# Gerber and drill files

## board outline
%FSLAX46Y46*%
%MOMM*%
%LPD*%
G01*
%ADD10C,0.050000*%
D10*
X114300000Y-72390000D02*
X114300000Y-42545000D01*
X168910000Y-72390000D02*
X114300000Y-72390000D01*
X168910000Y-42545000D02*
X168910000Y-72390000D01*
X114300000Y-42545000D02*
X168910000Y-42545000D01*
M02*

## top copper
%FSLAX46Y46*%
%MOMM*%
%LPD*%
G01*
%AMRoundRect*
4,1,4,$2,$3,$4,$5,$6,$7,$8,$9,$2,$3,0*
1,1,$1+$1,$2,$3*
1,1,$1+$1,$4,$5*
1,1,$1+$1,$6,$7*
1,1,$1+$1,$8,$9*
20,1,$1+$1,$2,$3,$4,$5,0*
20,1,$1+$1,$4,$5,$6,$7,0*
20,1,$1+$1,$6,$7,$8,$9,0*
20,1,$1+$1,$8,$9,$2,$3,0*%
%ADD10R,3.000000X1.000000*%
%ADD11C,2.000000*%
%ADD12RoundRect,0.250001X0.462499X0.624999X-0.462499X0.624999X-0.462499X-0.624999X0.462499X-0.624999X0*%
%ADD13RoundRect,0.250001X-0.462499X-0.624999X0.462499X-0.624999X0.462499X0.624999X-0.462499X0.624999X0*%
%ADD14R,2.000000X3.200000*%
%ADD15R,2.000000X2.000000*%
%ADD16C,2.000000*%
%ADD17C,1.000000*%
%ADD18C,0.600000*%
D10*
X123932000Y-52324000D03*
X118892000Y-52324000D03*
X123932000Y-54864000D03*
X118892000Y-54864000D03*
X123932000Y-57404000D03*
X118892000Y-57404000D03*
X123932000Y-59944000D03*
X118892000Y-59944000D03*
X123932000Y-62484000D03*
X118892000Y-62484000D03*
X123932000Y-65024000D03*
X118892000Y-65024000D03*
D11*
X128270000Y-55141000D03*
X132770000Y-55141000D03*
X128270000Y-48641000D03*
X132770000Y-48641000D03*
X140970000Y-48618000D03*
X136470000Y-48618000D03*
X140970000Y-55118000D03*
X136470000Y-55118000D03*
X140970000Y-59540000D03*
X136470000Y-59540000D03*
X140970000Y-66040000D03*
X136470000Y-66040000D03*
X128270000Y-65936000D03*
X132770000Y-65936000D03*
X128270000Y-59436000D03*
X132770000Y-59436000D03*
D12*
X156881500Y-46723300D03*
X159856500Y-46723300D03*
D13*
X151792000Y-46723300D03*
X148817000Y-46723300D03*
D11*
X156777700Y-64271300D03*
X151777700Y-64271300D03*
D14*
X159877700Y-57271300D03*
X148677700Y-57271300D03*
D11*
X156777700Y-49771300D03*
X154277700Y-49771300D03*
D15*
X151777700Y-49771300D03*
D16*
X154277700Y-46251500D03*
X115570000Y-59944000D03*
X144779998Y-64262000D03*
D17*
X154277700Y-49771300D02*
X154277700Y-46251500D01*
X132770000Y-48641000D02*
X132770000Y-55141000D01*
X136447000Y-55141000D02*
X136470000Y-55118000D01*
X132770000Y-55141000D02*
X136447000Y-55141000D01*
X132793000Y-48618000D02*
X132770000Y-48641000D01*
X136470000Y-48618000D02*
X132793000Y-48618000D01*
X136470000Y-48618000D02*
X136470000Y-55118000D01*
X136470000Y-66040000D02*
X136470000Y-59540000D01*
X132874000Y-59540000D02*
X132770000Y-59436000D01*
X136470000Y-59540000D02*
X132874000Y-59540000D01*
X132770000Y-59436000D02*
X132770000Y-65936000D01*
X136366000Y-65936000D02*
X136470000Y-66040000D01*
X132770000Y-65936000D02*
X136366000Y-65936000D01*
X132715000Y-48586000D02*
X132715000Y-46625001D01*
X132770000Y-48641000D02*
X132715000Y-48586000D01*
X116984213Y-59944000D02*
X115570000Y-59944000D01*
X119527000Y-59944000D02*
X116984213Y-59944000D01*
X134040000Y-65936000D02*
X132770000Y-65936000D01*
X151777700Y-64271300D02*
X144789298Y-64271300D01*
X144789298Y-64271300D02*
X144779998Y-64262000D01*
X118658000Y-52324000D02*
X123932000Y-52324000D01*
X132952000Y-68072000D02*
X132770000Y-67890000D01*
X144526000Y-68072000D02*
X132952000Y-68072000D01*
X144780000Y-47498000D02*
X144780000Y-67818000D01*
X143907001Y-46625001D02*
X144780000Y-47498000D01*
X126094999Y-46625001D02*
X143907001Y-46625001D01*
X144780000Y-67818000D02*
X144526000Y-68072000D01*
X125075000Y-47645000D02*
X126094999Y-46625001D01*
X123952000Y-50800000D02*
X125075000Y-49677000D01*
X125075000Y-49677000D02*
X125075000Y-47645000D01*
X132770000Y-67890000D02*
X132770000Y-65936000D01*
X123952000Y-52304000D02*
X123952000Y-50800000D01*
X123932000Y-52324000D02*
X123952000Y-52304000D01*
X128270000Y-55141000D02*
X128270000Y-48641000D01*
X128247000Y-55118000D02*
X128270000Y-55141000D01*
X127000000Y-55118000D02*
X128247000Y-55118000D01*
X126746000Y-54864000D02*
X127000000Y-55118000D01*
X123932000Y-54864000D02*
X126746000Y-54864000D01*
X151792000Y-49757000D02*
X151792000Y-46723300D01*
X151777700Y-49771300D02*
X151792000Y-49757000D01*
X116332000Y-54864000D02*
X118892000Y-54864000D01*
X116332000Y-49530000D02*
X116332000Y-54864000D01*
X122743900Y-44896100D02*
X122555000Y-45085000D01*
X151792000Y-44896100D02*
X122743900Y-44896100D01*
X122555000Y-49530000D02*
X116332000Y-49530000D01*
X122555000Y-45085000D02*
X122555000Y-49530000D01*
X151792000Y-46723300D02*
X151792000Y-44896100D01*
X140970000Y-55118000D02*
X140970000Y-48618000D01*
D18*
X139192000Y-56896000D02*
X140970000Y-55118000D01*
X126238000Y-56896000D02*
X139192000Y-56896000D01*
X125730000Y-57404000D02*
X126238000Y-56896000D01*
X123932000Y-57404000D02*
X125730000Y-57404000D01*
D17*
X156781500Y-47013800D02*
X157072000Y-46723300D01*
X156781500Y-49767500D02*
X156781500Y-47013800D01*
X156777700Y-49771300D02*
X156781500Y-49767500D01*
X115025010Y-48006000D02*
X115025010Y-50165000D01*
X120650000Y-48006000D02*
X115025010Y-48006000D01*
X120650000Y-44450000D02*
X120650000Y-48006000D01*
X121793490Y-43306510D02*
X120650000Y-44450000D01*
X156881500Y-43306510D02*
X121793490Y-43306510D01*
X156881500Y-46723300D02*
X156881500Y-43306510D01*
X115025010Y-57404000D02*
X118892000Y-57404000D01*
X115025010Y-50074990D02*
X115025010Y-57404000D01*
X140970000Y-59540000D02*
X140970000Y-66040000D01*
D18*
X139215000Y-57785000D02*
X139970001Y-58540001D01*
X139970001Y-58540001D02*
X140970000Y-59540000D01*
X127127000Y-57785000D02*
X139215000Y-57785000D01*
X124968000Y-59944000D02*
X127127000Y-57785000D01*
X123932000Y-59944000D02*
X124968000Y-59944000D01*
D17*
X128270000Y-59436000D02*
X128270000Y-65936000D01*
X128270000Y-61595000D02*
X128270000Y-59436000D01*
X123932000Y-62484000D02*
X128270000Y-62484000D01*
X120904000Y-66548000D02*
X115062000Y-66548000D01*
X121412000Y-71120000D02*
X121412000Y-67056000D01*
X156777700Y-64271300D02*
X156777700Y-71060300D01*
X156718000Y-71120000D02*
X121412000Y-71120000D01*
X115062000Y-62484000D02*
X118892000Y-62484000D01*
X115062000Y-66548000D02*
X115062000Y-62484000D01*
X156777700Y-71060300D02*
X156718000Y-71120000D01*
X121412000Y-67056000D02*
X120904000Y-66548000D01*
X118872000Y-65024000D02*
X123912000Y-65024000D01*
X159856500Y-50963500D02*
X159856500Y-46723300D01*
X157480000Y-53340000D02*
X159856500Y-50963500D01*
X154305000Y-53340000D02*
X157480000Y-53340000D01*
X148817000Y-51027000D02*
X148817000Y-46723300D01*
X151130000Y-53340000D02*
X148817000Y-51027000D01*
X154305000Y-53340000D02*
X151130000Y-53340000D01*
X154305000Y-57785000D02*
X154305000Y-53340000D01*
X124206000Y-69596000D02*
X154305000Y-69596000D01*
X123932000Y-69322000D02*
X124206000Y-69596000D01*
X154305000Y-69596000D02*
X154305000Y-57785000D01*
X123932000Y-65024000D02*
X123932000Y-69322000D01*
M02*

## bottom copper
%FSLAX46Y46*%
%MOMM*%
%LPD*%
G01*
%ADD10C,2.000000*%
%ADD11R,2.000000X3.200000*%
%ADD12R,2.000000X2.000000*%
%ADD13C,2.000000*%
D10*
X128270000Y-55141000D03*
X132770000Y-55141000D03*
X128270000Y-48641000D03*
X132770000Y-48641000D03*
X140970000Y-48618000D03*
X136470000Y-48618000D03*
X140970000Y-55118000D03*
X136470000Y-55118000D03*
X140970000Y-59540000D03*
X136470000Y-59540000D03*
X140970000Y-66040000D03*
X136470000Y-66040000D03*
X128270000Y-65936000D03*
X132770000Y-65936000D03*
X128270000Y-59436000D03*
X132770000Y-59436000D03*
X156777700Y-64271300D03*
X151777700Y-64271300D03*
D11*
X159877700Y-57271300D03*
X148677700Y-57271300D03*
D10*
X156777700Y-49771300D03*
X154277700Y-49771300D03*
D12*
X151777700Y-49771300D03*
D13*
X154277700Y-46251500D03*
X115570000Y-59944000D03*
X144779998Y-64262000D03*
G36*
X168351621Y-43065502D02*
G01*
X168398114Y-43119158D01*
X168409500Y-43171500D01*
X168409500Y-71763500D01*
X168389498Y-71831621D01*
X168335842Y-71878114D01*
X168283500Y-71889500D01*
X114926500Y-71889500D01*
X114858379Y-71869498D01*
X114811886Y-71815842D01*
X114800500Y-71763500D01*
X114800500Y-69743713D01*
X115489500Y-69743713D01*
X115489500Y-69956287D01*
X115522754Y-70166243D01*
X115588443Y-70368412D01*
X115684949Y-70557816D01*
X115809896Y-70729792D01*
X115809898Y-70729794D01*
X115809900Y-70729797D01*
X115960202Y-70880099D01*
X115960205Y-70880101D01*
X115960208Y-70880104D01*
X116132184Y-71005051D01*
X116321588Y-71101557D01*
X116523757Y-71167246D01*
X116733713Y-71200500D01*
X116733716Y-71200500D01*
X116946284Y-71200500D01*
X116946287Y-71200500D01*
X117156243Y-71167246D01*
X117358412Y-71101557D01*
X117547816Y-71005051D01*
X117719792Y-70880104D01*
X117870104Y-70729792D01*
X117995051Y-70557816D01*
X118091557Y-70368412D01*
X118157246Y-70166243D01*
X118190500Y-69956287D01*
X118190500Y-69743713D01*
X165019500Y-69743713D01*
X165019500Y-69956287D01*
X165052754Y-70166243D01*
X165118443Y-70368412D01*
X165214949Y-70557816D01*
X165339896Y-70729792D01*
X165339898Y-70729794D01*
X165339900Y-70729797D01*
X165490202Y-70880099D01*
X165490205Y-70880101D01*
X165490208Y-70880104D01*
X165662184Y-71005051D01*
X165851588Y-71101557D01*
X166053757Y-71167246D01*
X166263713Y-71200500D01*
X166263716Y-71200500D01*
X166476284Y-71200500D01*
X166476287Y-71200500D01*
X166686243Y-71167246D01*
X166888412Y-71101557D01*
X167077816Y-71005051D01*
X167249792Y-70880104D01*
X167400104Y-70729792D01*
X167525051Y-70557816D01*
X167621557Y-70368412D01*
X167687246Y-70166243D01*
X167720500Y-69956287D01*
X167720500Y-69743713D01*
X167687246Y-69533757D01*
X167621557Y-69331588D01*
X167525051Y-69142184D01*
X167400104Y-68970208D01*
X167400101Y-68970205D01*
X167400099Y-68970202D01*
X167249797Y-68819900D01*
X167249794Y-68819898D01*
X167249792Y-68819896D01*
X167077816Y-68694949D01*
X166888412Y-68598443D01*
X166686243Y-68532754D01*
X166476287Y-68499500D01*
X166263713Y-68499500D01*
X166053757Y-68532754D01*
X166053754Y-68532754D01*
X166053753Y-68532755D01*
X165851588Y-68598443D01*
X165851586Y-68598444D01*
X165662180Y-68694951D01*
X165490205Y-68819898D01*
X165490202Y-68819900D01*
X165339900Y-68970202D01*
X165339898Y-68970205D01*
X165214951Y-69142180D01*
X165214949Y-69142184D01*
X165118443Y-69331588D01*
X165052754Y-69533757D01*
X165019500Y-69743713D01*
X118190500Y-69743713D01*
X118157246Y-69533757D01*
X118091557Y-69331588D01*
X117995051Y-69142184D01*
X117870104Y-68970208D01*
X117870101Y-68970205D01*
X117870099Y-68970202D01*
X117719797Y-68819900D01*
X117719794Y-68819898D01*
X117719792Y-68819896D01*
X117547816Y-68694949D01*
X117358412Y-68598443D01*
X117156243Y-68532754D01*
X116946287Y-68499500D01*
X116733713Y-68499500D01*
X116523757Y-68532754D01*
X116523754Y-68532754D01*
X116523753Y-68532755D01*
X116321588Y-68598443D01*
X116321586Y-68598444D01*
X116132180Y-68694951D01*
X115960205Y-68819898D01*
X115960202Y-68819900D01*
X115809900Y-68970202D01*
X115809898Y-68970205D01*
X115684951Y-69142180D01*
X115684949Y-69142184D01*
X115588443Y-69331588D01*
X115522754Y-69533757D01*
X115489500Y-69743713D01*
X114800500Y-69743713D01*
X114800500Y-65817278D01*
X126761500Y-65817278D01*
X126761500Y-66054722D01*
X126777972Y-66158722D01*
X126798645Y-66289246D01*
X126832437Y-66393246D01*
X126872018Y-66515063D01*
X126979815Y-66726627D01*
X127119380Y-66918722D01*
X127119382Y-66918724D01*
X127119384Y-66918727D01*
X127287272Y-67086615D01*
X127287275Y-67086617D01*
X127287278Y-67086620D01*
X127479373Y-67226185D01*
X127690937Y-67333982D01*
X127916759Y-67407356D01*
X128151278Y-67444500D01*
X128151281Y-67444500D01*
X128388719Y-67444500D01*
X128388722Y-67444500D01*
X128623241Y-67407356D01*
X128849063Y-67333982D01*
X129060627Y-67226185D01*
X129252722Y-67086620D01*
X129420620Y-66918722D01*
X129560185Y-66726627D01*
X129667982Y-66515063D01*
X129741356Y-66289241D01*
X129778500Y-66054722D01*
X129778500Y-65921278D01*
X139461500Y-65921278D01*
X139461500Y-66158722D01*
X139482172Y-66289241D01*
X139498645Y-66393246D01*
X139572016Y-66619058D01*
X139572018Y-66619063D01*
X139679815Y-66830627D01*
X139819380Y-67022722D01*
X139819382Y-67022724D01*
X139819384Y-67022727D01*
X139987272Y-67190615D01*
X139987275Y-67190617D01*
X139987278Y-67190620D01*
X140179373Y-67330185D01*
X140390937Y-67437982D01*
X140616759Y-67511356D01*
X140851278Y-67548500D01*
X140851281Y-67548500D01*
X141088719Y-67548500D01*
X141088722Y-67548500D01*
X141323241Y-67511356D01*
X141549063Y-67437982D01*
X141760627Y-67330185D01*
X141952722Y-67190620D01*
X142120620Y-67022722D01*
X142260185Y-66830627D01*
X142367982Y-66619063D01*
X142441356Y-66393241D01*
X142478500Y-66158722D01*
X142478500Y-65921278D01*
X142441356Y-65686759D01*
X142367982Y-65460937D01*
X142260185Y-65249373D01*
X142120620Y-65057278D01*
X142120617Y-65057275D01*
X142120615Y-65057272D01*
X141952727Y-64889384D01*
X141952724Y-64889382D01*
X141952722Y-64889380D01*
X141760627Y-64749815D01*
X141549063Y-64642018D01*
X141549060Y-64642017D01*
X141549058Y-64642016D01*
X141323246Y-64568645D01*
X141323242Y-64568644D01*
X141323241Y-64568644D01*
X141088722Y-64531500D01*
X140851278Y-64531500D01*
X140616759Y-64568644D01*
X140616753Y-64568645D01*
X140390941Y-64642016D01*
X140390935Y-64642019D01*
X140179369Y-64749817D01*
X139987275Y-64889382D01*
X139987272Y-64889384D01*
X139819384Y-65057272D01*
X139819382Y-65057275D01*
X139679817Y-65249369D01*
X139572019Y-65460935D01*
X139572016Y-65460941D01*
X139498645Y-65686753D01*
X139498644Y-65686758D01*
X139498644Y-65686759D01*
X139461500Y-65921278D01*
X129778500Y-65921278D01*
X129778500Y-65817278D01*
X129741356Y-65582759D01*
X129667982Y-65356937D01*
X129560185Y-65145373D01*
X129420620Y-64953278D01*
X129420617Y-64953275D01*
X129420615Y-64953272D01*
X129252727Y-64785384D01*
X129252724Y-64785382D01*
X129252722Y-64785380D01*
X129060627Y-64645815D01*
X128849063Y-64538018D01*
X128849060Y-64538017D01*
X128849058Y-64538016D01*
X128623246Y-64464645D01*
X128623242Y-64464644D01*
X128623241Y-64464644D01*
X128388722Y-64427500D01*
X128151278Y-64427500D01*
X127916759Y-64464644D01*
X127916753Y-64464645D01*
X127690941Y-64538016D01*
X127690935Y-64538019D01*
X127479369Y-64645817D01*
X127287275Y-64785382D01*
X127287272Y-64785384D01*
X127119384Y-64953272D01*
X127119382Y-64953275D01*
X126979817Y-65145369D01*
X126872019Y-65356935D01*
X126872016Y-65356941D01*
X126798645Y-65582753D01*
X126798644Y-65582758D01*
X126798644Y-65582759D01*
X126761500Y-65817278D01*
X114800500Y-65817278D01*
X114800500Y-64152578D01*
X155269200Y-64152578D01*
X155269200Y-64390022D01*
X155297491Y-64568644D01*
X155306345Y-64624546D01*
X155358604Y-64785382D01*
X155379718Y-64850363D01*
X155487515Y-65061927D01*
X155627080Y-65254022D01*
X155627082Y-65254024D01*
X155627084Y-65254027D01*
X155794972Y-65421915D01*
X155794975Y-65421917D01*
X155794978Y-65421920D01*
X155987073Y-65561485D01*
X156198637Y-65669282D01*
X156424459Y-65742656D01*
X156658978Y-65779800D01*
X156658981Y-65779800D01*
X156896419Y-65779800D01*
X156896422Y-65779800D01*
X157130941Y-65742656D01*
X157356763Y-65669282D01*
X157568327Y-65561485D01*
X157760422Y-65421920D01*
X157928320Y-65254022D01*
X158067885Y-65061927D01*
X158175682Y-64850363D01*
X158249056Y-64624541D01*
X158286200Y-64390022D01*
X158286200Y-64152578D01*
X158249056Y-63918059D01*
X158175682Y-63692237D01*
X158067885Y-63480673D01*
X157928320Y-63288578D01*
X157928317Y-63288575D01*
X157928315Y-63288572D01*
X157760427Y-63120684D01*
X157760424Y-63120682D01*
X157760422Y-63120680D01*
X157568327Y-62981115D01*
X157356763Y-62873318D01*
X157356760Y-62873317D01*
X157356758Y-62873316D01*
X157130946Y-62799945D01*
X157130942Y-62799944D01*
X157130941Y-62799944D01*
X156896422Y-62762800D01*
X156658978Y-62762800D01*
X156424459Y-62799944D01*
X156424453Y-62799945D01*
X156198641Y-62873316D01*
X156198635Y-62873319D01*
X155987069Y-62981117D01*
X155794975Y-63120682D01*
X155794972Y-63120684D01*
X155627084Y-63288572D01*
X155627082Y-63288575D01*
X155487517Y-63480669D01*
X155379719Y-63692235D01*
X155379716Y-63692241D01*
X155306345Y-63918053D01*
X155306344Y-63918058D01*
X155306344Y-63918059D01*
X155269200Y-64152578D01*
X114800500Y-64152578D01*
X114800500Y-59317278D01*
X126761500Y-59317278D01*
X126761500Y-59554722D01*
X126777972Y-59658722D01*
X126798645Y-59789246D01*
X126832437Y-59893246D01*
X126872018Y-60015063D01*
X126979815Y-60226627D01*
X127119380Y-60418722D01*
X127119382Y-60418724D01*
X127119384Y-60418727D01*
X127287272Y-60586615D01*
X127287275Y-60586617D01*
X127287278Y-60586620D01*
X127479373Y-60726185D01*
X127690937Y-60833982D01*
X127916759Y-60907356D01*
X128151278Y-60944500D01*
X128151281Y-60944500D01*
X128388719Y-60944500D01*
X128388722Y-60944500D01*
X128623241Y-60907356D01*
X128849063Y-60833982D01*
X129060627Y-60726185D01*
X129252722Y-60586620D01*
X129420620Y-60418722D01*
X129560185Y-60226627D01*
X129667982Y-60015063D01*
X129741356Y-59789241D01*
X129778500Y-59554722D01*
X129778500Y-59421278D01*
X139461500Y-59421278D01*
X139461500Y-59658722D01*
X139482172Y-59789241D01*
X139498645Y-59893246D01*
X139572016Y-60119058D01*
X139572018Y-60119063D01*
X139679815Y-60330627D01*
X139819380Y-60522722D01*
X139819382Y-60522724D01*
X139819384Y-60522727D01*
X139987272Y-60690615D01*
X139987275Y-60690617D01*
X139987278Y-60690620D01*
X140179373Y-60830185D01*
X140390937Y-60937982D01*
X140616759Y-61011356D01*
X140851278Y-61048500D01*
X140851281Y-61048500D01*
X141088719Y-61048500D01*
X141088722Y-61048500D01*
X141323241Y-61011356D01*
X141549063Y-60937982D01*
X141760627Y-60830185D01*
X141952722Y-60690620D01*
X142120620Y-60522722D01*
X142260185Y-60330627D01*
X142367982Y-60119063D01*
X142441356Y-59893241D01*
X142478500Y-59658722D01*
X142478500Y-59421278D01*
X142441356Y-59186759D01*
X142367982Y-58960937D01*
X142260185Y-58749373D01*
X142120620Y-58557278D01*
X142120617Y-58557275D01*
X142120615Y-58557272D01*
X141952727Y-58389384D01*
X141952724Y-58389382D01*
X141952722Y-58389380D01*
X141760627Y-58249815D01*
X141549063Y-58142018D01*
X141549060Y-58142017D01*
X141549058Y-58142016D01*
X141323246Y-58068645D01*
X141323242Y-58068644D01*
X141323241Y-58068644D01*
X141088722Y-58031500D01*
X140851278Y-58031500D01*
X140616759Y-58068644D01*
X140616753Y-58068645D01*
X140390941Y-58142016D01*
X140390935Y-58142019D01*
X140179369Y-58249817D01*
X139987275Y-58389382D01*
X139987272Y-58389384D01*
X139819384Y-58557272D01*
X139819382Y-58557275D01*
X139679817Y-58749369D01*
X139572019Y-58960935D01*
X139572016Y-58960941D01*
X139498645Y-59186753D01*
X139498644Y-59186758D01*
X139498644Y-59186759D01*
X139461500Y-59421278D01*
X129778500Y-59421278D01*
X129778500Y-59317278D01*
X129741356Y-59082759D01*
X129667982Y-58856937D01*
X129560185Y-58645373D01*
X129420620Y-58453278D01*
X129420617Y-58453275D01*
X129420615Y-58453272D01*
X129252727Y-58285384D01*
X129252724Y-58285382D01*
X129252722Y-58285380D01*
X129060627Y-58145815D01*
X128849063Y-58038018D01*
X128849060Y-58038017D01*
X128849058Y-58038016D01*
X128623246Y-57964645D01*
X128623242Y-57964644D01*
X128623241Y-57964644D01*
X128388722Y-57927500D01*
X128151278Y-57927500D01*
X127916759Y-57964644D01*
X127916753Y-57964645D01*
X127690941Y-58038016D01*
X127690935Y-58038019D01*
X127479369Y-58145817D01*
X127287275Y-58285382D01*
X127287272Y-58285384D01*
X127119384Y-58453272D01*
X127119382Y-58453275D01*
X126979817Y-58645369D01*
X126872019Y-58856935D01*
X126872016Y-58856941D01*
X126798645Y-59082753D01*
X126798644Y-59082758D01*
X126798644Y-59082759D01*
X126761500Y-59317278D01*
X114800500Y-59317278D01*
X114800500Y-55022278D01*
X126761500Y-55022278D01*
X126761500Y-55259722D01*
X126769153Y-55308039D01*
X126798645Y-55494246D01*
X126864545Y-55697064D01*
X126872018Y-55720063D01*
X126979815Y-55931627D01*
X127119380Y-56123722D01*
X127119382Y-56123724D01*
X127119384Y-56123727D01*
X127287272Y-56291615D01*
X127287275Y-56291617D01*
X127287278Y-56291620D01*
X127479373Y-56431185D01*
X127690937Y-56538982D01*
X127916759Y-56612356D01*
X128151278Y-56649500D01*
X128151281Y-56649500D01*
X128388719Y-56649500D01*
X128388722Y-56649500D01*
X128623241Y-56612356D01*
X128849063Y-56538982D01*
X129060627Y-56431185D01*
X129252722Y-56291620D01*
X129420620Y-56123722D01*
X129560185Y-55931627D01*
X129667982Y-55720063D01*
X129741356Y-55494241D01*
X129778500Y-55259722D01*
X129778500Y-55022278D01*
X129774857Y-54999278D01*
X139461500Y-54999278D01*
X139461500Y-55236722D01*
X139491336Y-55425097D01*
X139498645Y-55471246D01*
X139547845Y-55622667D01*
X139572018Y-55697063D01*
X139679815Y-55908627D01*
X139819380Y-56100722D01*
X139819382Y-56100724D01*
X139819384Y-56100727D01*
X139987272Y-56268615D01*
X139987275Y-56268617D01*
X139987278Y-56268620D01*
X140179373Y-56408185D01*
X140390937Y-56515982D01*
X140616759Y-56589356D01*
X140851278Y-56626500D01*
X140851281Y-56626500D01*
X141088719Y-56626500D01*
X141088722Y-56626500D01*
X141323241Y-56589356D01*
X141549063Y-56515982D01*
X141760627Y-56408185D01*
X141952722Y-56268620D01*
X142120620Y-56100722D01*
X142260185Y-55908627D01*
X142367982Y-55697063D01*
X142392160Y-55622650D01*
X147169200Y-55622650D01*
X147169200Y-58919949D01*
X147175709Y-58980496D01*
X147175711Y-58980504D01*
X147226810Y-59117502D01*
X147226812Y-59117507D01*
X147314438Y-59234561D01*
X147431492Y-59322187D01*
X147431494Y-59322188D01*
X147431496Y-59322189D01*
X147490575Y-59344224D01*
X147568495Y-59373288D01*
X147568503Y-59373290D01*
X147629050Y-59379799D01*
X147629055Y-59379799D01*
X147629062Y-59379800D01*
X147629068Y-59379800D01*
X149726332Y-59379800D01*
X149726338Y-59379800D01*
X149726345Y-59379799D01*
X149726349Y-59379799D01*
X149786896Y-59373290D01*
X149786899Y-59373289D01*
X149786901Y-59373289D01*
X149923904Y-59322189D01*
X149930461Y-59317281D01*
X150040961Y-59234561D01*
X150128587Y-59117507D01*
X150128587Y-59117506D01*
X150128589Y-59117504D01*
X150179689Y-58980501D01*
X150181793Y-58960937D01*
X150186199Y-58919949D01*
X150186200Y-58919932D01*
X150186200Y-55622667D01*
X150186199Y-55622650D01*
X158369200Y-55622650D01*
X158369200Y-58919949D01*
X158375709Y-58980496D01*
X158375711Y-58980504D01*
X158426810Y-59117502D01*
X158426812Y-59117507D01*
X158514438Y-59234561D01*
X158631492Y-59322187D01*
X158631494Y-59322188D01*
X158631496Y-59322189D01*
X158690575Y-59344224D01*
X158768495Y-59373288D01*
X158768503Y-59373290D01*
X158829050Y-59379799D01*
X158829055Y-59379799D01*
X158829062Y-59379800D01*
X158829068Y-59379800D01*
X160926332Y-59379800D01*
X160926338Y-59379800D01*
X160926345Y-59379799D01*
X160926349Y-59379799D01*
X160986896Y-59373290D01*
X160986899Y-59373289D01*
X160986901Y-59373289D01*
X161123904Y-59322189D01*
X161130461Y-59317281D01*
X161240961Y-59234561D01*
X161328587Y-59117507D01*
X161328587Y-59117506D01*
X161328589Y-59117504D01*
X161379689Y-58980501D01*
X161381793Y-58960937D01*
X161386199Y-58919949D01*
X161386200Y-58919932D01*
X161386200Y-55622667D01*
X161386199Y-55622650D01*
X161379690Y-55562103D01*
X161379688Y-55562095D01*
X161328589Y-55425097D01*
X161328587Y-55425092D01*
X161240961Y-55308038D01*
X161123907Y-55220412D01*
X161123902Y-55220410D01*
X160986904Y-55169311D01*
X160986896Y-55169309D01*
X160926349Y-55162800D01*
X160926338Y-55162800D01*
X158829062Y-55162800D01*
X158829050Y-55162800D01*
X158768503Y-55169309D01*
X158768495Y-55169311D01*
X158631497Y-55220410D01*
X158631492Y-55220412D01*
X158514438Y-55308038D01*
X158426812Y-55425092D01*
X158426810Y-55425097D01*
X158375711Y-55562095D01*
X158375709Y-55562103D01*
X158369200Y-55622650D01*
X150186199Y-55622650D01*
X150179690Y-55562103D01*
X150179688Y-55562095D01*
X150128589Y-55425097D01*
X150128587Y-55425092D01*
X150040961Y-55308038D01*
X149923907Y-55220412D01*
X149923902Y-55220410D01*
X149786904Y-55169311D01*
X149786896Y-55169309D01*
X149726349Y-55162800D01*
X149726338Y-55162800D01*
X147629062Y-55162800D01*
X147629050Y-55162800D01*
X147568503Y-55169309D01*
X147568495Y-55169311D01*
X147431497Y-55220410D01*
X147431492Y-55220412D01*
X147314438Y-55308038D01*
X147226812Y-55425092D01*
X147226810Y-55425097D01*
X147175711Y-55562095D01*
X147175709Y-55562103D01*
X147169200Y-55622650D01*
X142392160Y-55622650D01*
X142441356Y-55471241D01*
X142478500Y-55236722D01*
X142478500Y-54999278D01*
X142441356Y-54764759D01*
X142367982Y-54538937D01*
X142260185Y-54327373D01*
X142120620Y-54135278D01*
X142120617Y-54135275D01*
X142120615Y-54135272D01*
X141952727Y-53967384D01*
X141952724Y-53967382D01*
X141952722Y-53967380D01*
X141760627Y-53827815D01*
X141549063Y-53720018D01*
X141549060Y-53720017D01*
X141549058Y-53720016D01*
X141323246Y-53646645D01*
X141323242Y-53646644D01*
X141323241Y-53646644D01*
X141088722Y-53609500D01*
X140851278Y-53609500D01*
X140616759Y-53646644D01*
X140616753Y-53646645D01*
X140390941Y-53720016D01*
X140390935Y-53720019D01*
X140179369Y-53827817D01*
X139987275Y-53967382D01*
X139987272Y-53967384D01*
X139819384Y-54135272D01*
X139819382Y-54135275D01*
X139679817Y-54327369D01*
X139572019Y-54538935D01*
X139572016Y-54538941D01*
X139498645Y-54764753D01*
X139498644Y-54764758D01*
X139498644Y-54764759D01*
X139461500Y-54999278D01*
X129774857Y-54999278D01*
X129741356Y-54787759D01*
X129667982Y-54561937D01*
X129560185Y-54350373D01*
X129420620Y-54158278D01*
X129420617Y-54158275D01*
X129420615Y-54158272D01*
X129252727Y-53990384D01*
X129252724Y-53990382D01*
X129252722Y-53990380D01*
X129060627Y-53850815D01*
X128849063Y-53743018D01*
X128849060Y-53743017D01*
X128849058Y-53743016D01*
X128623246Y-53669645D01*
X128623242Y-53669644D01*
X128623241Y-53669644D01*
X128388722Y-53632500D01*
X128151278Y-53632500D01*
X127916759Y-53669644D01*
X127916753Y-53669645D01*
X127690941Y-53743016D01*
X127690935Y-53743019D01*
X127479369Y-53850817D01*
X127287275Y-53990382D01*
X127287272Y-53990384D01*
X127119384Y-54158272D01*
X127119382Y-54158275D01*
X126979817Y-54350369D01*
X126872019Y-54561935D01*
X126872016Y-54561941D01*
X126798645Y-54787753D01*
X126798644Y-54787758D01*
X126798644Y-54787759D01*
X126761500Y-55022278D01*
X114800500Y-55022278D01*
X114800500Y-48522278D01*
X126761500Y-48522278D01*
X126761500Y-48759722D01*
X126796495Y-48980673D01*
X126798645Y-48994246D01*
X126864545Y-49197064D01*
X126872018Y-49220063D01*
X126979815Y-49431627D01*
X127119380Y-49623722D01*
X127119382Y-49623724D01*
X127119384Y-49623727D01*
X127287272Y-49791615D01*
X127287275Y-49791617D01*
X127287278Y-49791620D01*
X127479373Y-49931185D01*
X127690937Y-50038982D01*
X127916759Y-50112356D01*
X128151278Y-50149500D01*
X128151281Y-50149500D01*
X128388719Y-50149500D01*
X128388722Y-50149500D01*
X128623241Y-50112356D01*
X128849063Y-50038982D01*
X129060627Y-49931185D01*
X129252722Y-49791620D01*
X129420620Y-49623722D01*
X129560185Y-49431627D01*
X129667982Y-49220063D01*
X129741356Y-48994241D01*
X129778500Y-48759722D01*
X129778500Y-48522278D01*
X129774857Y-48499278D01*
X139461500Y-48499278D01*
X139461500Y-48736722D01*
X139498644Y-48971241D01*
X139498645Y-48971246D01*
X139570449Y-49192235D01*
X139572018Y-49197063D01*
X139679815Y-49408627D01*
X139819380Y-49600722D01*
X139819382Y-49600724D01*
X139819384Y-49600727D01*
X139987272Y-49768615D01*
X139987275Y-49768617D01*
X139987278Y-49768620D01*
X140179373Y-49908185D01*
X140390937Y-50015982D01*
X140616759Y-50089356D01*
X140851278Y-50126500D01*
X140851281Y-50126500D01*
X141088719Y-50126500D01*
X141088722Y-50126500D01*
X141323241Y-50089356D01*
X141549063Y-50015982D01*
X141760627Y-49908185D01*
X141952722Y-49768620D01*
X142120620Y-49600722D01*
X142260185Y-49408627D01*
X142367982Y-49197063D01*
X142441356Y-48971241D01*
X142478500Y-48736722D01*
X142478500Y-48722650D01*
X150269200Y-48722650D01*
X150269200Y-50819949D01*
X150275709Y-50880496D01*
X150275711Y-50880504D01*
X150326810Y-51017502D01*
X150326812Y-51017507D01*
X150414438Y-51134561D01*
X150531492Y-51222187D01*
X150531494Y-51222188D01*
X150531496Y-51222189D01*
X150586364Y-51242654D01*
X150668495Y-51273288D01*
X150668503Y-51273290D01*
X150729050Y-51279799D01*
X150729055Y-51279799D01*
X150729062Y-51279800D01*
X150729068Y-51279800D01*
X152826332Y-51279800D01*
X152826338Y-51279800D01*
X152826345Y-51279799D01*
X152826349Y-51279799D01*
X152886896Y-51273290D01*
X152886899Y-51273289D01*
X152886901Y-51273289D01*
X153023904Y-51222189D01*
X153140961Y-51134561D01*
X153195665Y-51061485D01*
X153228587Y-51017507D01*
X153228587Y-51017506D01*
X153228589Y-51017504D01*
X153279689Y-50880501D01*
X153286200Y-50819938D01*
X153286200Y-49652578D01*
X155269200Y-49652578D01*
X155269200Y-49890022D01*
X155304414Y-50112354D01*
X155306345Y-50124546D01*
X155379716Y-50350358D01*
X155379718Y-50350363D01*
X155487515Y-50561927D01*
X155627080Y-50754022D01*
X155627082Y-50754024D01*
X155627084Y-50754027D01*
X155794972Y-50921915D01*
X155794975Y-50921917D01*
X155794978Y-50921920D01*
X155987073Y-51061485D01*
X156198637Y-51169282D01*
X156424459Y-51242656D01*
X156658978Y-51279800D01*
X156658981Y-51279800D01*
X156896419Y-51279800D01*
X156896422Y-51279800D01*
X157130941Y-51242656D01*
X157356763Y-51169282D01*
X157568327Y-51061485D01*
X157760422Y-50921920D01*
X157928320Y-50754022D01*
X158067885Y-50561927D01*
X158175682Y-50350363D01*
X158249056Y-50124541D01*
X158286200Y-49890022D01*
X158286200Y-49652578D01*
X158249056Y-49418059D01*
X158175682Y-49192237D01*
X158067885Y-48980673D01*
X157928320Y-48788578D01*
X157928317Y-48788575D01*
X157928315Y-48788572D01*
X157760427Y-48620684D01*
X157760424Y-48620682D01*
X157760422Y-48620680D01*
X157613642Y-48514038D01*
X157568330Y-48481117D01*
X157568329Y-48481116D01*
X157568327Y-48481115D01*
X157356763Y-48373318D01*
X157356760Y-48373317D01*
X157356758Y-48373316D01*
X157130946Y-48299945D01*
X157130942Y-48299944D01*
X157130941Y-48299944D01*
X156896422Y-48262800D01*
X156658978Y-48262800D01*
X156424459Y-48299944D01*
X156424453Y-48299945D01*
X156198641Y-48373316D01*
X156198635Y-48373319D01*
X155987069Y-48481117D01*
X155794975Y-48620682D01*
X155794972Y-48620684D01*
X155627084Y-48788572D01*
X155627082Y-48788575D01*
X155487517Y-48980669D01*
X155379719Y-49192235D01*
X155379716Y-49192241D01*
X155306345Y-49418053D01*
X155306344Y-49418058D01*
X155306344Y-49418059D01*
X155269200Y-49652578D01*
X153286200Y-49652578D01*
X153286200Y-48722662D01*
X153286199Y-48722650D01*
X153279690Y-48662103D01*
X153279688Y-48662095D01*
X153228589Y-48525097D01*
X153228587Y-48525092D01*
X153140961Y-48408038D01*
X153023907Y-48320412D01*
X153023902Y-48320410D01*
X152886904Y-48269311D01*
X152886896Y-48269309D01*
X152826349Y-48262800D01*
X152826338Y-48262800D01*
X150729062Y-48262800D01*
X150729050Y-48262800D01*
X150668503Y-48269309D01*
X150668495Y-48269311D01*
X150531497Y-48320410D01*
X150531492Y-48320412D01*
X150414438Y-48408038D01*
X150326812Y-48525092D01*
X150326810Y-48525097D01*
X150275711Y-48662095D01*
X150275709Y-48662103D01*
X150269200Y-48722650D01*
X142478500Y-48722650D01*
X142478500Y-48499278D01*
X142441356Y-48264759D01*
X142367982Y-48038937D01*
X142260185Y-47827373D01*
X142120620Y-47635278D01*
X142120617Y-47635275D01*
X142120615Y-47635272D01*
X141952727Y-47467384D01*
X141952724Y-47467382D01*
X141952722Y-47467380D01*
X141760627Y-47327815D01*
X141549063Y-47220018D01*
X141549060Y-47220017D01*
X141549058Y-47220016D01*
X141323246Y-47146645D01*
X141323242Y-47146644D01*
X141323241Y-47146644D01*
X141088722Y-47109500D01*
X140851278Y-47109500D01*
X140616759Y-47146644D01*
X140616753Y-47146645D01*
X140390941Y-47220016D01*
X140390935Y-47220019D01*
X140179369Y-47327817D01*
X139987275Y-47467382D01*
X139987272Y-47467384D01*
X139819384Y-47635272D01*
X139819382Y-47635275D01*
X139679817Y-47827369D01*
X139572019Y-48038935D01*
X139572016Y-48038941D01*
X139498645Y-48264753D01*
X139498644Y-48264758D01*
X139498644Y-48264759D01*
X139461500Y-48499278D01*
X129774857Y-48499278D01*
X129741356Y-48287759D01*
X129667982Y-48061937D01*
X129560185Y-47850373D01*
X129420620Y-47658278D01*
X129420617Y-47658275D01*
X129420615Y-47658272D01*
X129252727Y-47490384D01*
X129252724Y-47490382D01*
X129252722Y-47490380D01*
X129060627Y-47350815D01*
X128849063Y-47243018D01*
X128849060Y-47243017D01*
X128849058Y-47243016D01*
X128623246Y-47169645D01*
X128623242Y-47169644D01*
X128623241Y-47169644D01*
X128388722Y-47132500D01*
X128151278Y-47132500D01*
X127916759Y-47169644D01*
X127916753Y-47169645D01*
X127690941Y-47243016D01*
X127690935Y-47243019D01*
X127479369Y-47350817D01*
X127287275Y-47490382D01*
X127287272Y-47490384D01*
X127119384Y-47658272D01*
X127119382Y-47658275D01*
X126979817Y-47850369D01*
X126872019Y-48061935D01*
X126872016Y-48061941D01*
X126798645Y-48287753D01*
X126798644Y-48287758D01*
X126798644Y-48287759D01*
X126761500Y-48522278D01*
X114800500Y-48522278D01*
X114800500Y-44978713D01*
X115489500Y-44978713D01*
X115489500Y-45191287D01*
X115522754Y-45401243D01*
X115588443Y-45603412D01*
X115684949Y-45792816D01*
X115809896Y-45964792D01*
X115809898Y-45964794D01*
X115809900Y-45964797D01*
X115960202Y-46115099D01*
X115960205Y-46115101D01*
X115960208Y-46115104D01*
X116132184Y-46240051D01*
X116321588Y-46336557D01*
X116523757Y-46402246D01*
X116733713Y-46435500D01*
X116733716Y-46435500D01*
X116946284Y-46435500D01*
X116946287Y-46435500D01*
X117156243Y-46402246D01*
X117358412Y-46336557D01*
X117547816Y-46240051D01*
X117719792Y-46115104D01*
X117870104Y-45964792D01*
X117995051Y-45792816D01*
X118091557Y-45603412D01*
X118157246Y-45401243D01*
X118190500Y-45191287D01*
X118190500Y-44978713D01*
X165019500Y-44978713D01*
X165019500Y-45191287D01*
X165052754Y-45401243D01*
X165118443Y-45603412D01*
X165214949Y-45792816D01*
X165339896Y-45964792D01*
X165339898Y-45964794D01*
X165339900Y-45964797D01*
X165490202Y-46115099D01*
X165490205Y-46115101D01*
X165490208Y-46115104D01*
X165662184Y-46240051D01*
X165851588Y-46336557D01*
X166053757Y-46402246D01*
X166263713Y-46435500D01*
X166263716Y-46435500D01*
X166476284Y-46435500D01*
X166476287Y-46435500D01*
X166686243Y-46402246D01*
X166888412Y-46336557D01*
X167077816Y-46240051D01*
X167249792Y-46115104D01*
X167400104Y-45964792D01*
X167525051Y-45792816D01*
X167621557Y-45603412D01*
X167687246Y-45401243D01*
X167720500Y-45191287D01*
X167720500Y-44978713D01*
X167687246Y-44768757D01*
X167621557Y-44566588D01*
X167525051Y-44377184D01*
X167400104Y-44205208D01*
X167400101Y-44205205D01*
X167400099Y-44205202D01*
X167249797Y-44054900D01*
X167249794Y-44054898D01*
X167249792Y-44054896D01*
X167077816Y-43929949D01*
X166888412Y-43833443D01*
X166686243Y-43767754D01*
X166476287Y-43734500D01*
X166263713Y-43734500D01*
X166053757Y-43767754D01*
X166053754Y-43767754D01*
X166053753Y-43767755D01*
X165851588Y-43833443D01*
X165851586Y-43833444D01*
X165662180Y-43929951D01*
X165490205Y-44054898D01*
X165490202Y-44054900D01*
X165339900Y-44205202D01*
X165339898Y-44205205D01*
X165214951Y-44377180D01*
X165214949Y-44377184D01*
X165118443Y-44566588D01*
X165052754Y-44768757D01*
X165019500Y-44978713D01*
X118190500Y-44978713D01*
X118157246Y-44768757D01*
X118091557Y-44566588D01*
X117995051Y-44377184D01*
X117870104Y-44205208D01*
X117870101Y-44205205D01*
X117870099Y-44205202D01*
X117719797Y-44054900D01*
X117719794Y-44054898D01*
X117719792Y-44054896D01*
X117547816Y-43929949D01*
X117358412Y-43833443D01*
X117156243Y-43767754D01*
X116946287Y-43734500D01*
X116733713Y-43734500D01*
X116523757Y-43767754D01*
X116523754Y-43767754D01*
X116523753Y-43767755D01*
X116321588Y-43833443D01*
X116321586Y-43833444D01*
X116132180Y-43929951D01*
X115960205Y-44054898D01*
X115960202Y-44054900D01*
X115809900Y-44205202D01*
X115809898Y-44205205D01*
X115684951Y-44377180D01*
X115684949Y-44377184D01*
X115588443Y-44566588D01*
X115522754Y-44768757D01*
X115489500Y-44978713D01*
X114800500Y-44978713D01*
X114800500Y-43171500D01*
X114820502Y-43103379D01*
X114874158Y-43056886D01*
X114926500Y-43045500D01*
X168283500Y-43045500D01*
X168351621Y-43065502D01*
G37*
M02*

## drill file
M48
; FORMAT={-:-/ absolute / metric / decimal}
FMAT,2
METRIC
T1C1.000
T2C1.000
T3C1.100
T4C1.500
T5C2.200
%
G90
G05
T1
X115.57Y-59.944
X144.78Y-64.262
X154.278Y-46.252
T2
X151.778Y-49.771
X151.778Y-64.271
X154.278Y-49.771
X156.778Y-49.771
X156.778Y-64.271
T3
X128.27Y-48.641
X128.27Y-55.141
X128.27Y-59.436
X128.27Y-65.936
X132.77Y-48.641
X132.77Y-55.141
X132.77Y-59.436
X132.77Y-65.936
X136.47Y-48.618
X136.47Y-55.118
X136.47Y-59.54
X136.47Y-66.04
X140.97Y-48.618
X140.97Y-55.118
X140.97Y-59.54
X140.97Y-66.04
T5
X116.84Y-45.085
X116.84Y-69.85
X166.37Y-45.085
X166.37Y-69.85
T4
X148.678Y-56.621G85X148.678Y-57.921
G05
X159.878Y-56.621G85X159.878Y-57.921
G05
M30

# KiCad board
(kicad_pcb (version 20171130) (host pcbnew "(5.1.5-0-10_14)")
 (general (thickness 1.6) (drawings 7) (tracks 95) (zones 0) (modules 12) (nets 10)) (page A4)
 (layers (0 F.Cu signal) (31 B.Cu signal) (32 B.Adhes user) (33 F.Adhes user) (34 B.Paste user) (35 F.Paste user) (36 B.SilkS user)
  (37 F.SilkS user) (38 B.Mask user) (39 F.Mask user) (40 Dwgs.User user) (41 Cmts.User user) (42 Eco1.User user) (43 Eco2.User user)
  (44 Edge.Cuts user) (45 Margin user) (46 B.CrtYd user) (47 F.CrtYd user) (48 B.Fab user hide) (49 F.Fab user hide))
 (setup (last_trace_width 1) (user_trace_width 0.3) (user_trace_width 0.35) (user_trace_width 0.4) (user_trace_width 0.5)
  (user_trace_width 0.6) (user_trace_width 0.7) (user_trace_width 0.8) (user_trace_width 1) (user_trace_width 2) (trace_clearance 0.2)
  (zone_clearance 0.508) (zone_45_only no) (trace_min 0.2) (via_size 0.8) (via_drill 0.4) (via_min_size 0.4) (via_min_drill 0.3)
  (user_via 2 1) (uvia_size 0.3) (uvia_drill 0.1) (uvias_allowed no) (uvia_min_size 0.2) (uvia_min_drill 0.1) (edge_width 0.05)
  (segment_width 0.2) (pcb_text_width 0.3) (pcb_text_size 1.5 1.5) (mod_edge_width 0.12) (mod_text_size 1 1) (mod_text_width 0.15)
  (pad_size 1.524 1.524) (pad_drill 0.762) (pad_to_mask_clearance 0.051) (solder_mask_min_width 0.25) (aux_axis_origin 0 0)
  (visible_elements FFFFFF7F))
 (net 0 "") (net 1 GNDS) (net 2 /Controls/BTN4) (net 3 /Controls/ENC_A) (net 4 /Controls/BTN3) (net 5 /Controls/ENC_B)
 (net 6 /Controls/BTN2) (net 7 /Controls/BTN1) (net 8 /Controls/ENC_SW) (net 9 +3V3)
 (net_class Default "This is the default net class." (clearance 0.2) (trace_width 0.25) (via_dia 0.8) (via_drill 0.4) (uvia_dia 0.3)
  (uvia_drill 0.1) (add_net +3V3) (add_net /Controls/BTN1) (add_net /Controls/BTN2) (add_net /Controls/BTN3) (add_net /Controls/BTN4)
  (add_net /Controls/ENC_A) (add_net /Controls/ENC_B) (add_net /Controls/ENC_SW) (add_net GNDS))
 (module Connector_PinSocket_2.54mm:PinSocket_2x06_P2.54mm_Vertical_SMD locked (layer F.Cu) (at 121.412 58.674 180)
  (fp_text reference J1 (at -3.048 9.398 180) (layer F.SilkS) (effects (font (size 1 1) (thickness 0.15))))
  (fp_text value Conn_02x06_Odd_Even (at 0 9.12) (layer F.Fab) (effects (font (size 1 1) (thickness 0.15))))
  (pad 12 smd rect (at -2.52 6.35 180) (size 3 1) (layers F.Cu F.Paste F.Mask) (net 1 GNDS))
  (pad 11 smd rect (at 2.52 6.35 180) (size 3 1) (layers F.Cu F.Paste F.Mask) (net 1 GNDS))
  (pad 10 smd rect (at -2.52 3.81 180) (size 3 1) (layers F.Cu F.Paste F.Mask) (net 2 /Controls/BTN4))
  (pad 9 smd rect (at 2.52 3.81 180) (size 3 1) (layers F.Cu F.Paste F.Mask) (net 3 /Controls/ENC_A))
  (pad 8 smd rect (at -2.52 1.27 180) (size 3 1) (layers F.Cu F.Paste F.Mask) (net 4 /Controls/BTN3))
  (pad 7 smd rect (at 2.52 1.27 180) (size 3 1) (layers F.Cu F.Paste F.Mask) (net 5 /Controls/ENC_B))
  (pad 6 smd rect (at -2.52 -1.27 180) (size 3 1) (layers F.Cu F.Paste F.Mask) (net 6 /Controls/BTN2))
  (pad 5 smd rect (at 2.52 -1.27 180) (size 3 1) (layers F.Cu F.Paste F.Mask) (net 1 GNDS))
  (pad 4 smd rect (at -2.52 -3.81 180) (size 3 1) (layers F.Cu F.Paste F.Mask) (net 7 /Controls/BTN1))
  (pad 3 smd rect (at 2.52 -3.81 180) (size 3 1) (layers F.Cu F.Paste F.Mask) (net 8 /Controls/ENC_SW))
  (pad 2 smd rect (at -2.52 -6.35 180) (size 3 1) (layers F.Cu F.Paste F.Mask) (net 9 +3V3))
  (pad 1 smd rect (at 2.52 -6.35 180) (size 3 1) (layers F.Cu F.Paste F.Mask) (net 9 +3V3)))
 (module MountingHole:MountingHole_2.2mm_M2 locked (layer F.Cu) (at 166.37 45.085)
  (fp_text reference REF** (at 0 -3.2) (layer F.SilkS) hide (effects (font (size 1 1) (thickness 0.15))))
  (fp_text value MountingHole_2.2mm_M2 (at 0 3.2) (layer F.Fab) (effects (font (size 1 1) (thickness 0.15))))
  (pad 1 np_thru_hole circle (at 0 0) (size 2.2 2.2) (drill 2.2) (layers *.Cu *.Mask)))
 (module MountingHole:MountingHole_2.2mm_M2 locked (layer F.Cu) (at 166.37 69.85)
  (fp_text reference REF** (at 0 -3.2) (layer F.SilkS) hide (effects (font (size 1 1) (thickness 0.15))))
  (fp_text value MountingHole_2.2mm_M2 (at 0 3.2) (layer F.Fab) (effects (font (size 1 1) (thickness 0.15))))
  (pad 1 np_thru_hole circle (at 0 0) (size 2.2 2.2) (drill 2.2) (layers *.Cu *.Mask)))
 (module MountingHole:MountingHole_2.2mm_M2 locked (layer F.Cu) (at 116.84 69.85)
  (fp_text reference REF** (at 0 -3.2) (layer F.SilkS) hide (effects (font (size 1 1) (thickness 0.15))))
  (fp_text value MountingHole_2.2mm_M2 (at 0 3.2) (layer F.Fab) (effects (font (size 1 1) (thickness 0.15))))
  (pad 1 np_thru_hole circle (at 0 0) (size 2.2 2.2) (drill 2.2) (layers *.Cu *.Mask)))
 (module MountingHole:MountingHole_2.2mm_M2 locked (layer F.Cu) (at 116.84 45.085)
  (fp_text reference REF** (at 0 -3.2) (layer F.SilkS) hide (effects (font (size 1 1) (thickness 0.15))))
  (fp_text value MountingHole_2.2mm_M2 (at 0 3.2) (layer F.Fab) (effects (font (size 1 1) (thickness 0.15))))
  (pad 1 np_thru_hole circle (at 0 0) (size 2.2 2.2) (drill 2.2) (layers *.Cu *.Mask)))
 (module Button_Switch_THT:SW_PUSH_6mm (layer B.Cu) (at 128.27 48.641 270)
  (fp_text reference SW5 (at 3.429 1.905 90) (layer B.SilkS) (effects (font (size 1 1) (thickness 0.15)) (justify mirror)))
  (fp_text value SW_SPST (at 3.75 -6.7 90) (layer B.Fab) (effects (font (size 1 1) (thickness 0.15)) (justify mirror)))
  (pad 1 thru_hole circle (at 6.5 0 180) (size 2 2) (drill 1.1) (layers *.Cu *.Mask) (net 2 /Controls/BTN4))
  (pad 2 thru_hole circle (at 6.5 -4.5 180) (size 2 2) (drill 1.1) (layers *.Cu *.Mask) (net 1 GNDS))
  (pad 1 thru_hole circle (at 0 0 180) (size 2 2) (drill 1.1) (layers *.Cu *.Mask) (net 2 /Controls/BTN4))
  (pad 2 thru_hole circle (at 0 -4.5 180) (size 2 2) (drill 1.1) (layers *.Cu *.Mask) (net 1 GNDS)))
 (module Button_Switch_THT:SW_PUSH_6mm (layer B.Cu) (at 140.97 55.118 90)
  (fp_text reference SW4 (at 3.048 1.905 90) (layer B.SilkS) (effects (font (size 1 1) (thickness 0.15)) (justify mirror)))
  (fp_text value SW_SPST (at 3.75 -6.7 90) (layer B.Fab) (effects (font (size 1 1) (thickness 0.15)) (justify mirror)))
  (pad 1 thru_hole circle (at 6.5 0) (size 2 2) (drill 1.1) (layers *.Cu *.Mask) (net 4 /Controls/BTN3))
  (pad 2 thru_hole circle (at 6.5 -4.5) (size 2 2) (drill 1.1) (layers *.Cu *.Mask) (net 1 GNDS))
  (pad 1 thru_hole circle (at 0 0) (size 2 2) (drill 1.1) (layers *.Cu *.Mask) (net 4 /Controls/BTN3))
  (pad 2 thru_hole circle (at 0 -4.5) (size 2 2) (drill 1.1) (layers *.Cu *.Mask) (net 1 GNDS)))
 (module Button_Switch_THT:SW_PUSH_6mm (layer B.Cu) (at 140.97 66.04 90)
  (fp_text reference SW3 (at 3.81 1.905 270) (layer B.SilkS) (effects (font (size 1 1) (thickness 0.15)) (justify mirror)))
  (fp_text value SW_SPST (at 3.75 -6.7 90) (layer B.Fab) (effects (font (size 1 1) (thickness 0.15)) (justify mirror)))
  (pad 1 thru_hole circle (at 6.5 0) (size 2 2) (drill 1.1) (layers *.Cu *.Mask) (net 6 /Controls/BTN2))
  (pad 2 thru_hole circle (at 6.5 -4.5) (size 2 2) (drill 1.1) (layers *.Cu *.Mask) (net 1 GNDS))
  (pad 1 thru_hole circle (at 0 0) (size 2 2) (drill 1.1) (layers *.Cu *.Mask) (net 6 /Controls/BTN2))
  (pad 2 thru_hole circle (at 0 -4.5) (size 2 2) (drill 1.1) (layers *.Cu *.Mask) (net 1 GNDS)))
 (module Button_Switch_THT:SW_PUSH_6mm (layer B.Cu) (at 128.27 59.436 270)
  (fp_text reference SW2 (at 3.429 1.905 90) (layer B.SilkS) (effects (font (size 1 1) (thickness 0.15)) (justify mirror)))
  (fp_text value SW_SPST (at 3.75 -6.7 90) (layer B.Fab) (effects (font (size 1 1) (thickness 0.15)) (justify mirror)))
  (pad 1 thru_hole circle (at 6.5 0 180) (size 2 2) (drill 1.1) (layers *.Cu *.Mask) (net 7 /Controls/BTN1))
  (pad 2 thru_hole circle (at 6.5 -4.5 180) (size 2 2) (drill 1.1) (layers *.Cu *.Mask) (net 1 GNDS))
  (pad 1 thru_hole circle (at 0 0 180) (size 2 2) (drill 1.1) (layers *.Cu *.Mask) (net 7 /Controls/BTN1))
  (pad 2 thru_hole circle (at 0 -4.5 180) (size 2 2) (drill 1.1) (layers *.Cu *.Mask) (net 1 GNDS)))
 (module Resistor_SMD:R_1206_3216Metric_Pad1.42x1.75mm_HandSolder (layer F.Cu) (at 158.369 46.7233 180)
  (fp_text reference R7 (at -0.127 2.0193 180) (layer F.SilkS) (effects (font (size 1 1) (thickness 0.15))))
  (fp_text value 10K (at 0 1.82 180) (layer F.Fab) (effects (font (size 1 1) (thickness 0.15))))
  (pad 2 smd roundrect (at 1.4875 0 180) (size 1.425 1.75) (layers F.Cu F.Paste F.Mask) (roundrect_rratio 0.175439) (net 5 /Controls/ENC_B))
  (pad 1 smd roundrect (at -1.4875 0 180) (size 1.425 1.75) (layers F.Cu F.Paste F.Mask) (roundrect_rratio 0.175439) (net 9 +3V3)))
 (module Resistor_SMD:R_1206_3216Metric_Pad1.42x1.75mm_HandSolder (layer F.Cu) (at 150.3045 46.7233)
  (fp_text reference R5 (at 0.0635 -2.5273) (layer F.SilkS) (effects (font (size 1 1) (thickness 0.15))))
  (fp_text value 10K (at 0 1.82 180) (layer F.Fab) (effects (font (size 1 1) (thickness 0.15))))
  (pad 2 smd roundrect (at 1.4875 0) (size 1.425 1.75) (layers F.Cu F.Paste F.Mask) (roundrect_rratio 0.175439) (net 3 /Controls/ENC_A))
  (pad 1 smd roundrect (at -1.4875 0) (size 1.425 1.75) (layers F.Cu F.Paste F.Mask) (roundrect_rratio 0.175439) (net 9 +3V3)))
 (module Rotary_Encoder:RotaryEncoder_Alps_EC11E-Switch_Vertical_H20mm (layer B.Cu) (at 151.7777 49.7713 270)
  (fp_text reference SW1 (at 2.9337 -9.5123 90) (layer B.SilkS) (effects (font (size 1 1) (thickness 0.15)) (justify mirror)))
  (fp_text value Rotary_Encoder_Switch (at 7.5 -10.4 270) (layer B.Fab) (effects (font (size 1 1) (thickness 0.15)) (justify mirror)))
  (pad S1 thru_hole circle (at 14.5 -5 270) (size 2 2) (drill 1) (layers *.Cu *.Mask) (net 8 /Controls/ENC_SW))
  (pad S2 thru_hole circle (at 14.5 0 270) (size 2 2) (drill 1) (layers *.Cu *.Mask) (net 1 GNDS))
  (pad MP thru_hole rect (at 7.5 -8.1 270) (size 3.2 2) (drill oval 2.8 1.5) (layers *.Cu *.Mask))
  (pad MP thru_hole rect (at 7.5 3.1 270) (size 3.2 2) (drill oval 2.8 1.5) (layers *.Cu *.Mask))
  (pad B thru_hole circle (at 0 -5 270) (size 2 2) (drill 1) (layers *.Cu *.Mask) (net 5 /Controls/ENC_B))
  (pad C thru_hole circle (at 0 -2.5 270) (size 2 2) (drill 1) (layers *.Cu *.Mask) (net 1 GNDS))
  (pad A thru_hole rect (at 0 0 270) (size 2 2) (drill 1) (layers *.Cu *.Mask) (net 3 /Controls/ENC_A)))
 (gr_line (start 114.3 72.39) (end 114.3 42.545) (layer Edge.Cuts) (width 0.05))
 (gr_line (start 168.91 72.39) (end 114.3 72.39) (layer Edge.Cuts) (width 0.05))
 (gr_line (start 168.91 42.545) (end 168.91 72.39) (layer Edge.Cuts) (width 0.05))
 (gr_line (start 114.3 42.545) (end 168.91 42.545) (layer Edge.Cuts) (width 0.05))
 (segment (start 154.2777 49.7713) (end 154.2777 46.2515) (width 1) (layer F.Cu) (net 1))
 (via (at 154.2777 46.2515) (size 2) (drill 1) (layers F.Cu B.Cu) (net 1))
 (segment (start 132.77 48.641) (end 132.77 55.141) (width 1) (layer F.Cu) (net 1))
 (segment (start 136.447 55.141) (end 136.47 55.118) (width 1) (layer F.Cu) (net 1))
 (segment (start 132.77 55.141) (end 136.447 55.141) (width 1) (layer F.Cu) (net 1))
 (segment (start 132.793 48.618) (end 132.77 48.641) (width 1) (layer F.Cu) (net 1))
 (segment (start 136.47 48.618) (end 132.793 48.618) (width 1) (layer F.Cu) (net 1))
 (segment (start 136.47 48.618) (end 136.47 55.118) (width 1) (layer F.Cu) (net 1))
 (segment (start 136.47 66.04) (end 136.47 59.54) (width 1) (layer F.Cu) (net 1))
 (segment (start 132.874 59.54) (end 132.77 59.436) (width 1) (layer F.Cu) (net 1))
 (segment (start 136.47 59.54) (end 132.874 59.54) (width 1) (layer F.Cu) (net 1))
 (segment (start 132.77 59.436) (end 132.77 65.936) (width 1) (layer F.Cu) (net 1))
 (segment (start 136.366 65.936) (end 136.47 66.04) (width 1) (layer F.Cu) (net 1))
 (segment (start 132.77 65.936) (end 136.366 65.936) (width 1) (layer F.Cu) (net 1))
 (segment (start 132.715 48.586) (end 132.715 46.625001) (width 1) (layer F.Cu) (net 1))
 (segment (start 132.77 48.641) (end 132.715 48.586) (width 1) (layer F.Cu) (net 1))
 (segment (start 116.984213 59.944) (end 115.57 59.944) (width 1) (layer F.Cu) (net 1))
 (segment (start 119.527 59.944) (end 116.984213 59.944) (width 1) (layer F.Cu) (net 1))
 (via (at 115.57 59.944) (size 2) (drill 1) (layers F.Cu B.Cu) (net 1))
 (segment (start 134.04 65.936) (end 132.77 65.936) (width 1) (layer F.Cu) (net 1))
 (via (at 144.779998 64.262) (size 2) (drill 1) (layers F.Cu B.Cu) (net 1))
 (segment (start 151.7777 64.2713) (end 144.789298 64.2713) (width 1) (layer F.Cu) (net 1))
 (segment (start 144.789298 64.2713) (end 144.779998 64.262) (width 1) (layer F.Cu) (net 1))
 (segment (start 118.658 52.324) (end 123.932 52.324) (width 1) (layer F.Cu) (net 1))
 (segment (start 132.952 68.072) (end 132.77 67.89) (width 1) (layer F.Cu) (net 1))
 (segment (start 144.526 68.072) (end 132.952 68.072) (width 1) (layer F.Cu) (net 1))
 (segment (start 144.78 47.498) (end 144.78 67.818) (width 1) (layer F.Cu) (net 1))
 (segment (start 143.907001 46.625001) (end 144.78 47.498) (width 1) (layer F.Cu) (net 1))
 (segment (start 126.094999 46.625001) (end 143.907001 46.625001) (width 1) (layer F.Cu) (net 1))
 (segment (start 144.78 67.818) (end 144.526 68.072) (width 1) (layer F.Cu) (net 1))
 (segment (start 125.075 47.645) (end 126.094999 46.625001) (width 1) (layer F.Cu) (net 1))
 (segment (start 123.952 50.8) (end 125.075 49.677) (width 1) (layer F.Cu) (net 1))
 (segment (start 125.075 49.677) (end 125.075 47.645) (width 1) (layer F.Cu) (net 1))
 (segment (start 132.77 67.89) (end 132.77 65.936) (width 1) (layer F.Cu) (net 1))
 (segment (start 123.952 52.304) (end 123.952 50.8) (width 1) (layer F.Cu) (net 1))
 (segment (start 123.932 52.324) (end 123.952 52.304) (width 1) (layer F.Cu) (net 1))
 (segment (start 128.27 55.141) (end 128.27 48.641) (width 1) (layer F.Cu) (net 2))
 (segment (start 128.247 55.118) (end 128.27 55.141) (width 1) (layer F.Cu) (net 2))
 (segment (start 127 55.118) (end 128.247 55.118) (width 1) (layer F.Cu) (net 2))
 (segment (start 126.746 54.864) (end 127 55.118) (width 1) (layer F.Cu) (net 2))
 (segment (start 123.932 54.864) (end 126.746 54.864) (width 1) (layer F.Cu) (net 2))
 (segment (start 151.792 49.757) (end 151.792 46.7233) (width 1) (layer F.Cu) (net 3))
 (segment (start 151.7777 49.7713) (end 151.792 49.757) (width 1) (layer F.Cu) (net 3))
 (segment (start 116.332 54.864) (end 118.892 54.864) (width 1) (layer F.Cu) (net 3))
 (segment (start 116.332 49.53) (end 116.332 54.864) (width 1) (layer F.Cu) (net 3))
 (segment (start 122.7439 44.8961) (end 122.555 45.085) (width 1) (layer F.Cu) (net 3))
 (segment (start 151.792 44.8961) (end 122.7439 44.8961) (width 1) (layer F.Cu) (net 3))
 (segment (start 122.555 49.53) (end 116.332 49.53) (width 1) (layer F.Cu) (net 3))
 (segment (start 122.555 45.085) (end 122.555 49.53) (width 1) (layer F.Cu) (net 3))
 (segment (start 151.792 46.7233) (end 151.792 44.8961) (width 1) (layer F.Cu) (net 3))
 (segment (start 140.97 55.118) (end 140.97 48.618) (width 1) (layer F.Cu) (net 4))
 (segment (start 139.192 56.896) (end 140.97 55.118) (width 0.6) (layer F.Cu) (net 4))
 (segment (start 126.238 56.896) (end 139.192 56.896) (width 0.6) (layer F.Cu) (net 4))
 (segment (start 125.73 57.404) (end 126.238 56.896) (width 0.6) (layer F.Cu) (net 4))
 (segment (start 123.932 57.404) (end 125.73 57.404) (width 0.6) (layer F.Cu) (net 4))
 (segment (start 156.7815 47.0138) (end 157.072 46.7233) (width 1) (layer F.Cu) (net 5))
 (segment (start 156.7815 49.7675) (end 156.7815 47.0138) (width 1) (layer F.Cu) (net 5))
 (segment (start 156.7777 49.7713) (end 156.7815 49.7675) (width 1) (layer F.Cu) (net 5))
 (segment (start 115.02501 48.006) (end 115.02501 50.165) (width 1) (layer F.Cu) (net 5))
 (segment (start 120.65 48.006) (end 115.02501 48.006) (width 1) (layer F.Cu) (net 5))
 (segment (start 120.65 44.45) (end 120.65 48.006) (width 1) (layer F.Cu) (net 5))
 (segment (start 121.79349 43.30651) (end 120.65 44.45) (width 1) (layer F.Cu) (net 5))
 (segment (start 156.8815 43.30651) (end 121.79349 43.30651) (width 1) (layer F.Cu) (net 5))
 (segment (start 156.8815 46.7233) (end 156.8815 43.30651) (width 1) (layer F.Cu) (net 5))
 (segment (start 115.02501 57.404) (end 118.892 57.404) (width 1) (layer F.Cu) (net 5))
 (segment (start 115.02501 50.07499) (end 115.02501 57.404) (width 1) (layer F.Cu) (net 5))
 (segment (start 140.97 59.54) (end 140.97 66.04) (width 1) (layer F.Cu) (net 6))
 (segment (start 139.215 57.785) (end 139.970001 58.540001) (width 0.6) (layer F.Cu) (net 6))
 (segment (start 139.970001 58.540001) (end 140.97 59.54) (width 0.6) (layer F.Cu) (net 6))
 (segment (start 127.127 57.785) (end 139.215 57.785) (width 0.6) (layer F.Cu) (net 6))
 (segment (start 124.968 59.944) (end 127.127 57.785) (width 0.6) (layer F.Cu) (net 6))
 (segment (start 123.932 59.944) (end 124.968 59.944) (width 0.6) (layer F.Cu) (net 6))
 (segment (start 128.27 59.436) (end 128.27 65.936) (width 1) (layer F.Cu) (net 7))
 (segment (start 128.27 61.595) (end 128.27 59.436) (width 1) (layer F.Cu) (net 7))
 (segment (start 123.932 62.484) (end 128.27 62.484) (width 1) (layer F.Cu) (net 7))
 (segment (start 120.904 66.548) (end 115.062 66.548) (width 1) (layer F.Cu) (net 8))
 (segment (start 121.412 71.12) (end 121.412 67.056) (width 1) (layer F.Cu) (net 8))
 (segment (start 156.7777 64.2713) (end 156.7777 71.0603) (width 1) (layer F.Cu) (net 8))
 (segment (start 156.718 71.12) (end 121.412 71.12) (width 1) (layer F.Cu) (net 8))
 (segment (start 115.062 62.484) (end 118.892 62.484) (width 1) (layer F.Cu) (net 8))
 (segment (start 115.062 66.548) (end 115.062 62.484) (width 1) (layer F.Cu) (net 8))
 (segment (start 156.7777 71.0603) (end 156.718 71.12) (width 1) (layer F.Cu) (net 8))
 (segment (start 121.412 67.056) (end 120.904 66.548) (width 1) (layer F.Cu) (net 8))
 (segment (start 118.872 65.024) (end 123.912 65.024) (width 1) (layer F.Cu) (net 9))
 (segment (start 159.8565 50.9635) (end 159.8565 46.7233) (width 1) (layer F.Cu) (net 9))
 (segment (start 157.48 53.34) (end 159.8565 50.9635) (width 1) (layer F.Cu) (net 9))
 (segment (start 154.305 53.34) (end 157.48 53.34) (width 1) (layer F.Cu) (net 9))
 (segment (start 148.817 51.027) (end 148.817 46.7233) (width 1) (layer F.Cu) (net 9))
 (segment (start 151.13 53.34) (end 148.817 51.027) (width 1) (layer F.Cu) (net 9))
 (segment (start 154.305 53.34) (end 151.13 53.34) (width 1) (layer F.Cu) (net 9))
 (segment (start 154.305 57.785) (end 154.305 53.34) (width 1) (layer F.Cu) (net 9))
 (segment (start 124.206 69.596) (end 154.305 69.596) (width 1) (layer F.Cu) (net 9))
 (segment (start 123.932 69.322) (end 124.206 69.596) (width 1) (layer F.Cu) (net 9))
 (segment (start 154.305 69.596) (end 154.305 57.785) (width 1) (layer F.Cu) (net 9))
 (segment (start 123.932 65.024) (end 123.932 69.322) (width 1) (layer F.Cu) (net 9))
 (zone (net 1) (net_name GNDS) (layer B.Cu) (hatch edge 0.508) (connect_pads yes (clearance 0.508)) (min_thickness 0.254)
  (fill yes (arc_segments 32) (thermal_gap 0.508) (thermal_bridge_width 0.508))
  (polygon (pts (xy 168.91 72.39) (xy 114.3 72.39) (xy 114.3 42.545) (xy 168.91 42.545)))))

